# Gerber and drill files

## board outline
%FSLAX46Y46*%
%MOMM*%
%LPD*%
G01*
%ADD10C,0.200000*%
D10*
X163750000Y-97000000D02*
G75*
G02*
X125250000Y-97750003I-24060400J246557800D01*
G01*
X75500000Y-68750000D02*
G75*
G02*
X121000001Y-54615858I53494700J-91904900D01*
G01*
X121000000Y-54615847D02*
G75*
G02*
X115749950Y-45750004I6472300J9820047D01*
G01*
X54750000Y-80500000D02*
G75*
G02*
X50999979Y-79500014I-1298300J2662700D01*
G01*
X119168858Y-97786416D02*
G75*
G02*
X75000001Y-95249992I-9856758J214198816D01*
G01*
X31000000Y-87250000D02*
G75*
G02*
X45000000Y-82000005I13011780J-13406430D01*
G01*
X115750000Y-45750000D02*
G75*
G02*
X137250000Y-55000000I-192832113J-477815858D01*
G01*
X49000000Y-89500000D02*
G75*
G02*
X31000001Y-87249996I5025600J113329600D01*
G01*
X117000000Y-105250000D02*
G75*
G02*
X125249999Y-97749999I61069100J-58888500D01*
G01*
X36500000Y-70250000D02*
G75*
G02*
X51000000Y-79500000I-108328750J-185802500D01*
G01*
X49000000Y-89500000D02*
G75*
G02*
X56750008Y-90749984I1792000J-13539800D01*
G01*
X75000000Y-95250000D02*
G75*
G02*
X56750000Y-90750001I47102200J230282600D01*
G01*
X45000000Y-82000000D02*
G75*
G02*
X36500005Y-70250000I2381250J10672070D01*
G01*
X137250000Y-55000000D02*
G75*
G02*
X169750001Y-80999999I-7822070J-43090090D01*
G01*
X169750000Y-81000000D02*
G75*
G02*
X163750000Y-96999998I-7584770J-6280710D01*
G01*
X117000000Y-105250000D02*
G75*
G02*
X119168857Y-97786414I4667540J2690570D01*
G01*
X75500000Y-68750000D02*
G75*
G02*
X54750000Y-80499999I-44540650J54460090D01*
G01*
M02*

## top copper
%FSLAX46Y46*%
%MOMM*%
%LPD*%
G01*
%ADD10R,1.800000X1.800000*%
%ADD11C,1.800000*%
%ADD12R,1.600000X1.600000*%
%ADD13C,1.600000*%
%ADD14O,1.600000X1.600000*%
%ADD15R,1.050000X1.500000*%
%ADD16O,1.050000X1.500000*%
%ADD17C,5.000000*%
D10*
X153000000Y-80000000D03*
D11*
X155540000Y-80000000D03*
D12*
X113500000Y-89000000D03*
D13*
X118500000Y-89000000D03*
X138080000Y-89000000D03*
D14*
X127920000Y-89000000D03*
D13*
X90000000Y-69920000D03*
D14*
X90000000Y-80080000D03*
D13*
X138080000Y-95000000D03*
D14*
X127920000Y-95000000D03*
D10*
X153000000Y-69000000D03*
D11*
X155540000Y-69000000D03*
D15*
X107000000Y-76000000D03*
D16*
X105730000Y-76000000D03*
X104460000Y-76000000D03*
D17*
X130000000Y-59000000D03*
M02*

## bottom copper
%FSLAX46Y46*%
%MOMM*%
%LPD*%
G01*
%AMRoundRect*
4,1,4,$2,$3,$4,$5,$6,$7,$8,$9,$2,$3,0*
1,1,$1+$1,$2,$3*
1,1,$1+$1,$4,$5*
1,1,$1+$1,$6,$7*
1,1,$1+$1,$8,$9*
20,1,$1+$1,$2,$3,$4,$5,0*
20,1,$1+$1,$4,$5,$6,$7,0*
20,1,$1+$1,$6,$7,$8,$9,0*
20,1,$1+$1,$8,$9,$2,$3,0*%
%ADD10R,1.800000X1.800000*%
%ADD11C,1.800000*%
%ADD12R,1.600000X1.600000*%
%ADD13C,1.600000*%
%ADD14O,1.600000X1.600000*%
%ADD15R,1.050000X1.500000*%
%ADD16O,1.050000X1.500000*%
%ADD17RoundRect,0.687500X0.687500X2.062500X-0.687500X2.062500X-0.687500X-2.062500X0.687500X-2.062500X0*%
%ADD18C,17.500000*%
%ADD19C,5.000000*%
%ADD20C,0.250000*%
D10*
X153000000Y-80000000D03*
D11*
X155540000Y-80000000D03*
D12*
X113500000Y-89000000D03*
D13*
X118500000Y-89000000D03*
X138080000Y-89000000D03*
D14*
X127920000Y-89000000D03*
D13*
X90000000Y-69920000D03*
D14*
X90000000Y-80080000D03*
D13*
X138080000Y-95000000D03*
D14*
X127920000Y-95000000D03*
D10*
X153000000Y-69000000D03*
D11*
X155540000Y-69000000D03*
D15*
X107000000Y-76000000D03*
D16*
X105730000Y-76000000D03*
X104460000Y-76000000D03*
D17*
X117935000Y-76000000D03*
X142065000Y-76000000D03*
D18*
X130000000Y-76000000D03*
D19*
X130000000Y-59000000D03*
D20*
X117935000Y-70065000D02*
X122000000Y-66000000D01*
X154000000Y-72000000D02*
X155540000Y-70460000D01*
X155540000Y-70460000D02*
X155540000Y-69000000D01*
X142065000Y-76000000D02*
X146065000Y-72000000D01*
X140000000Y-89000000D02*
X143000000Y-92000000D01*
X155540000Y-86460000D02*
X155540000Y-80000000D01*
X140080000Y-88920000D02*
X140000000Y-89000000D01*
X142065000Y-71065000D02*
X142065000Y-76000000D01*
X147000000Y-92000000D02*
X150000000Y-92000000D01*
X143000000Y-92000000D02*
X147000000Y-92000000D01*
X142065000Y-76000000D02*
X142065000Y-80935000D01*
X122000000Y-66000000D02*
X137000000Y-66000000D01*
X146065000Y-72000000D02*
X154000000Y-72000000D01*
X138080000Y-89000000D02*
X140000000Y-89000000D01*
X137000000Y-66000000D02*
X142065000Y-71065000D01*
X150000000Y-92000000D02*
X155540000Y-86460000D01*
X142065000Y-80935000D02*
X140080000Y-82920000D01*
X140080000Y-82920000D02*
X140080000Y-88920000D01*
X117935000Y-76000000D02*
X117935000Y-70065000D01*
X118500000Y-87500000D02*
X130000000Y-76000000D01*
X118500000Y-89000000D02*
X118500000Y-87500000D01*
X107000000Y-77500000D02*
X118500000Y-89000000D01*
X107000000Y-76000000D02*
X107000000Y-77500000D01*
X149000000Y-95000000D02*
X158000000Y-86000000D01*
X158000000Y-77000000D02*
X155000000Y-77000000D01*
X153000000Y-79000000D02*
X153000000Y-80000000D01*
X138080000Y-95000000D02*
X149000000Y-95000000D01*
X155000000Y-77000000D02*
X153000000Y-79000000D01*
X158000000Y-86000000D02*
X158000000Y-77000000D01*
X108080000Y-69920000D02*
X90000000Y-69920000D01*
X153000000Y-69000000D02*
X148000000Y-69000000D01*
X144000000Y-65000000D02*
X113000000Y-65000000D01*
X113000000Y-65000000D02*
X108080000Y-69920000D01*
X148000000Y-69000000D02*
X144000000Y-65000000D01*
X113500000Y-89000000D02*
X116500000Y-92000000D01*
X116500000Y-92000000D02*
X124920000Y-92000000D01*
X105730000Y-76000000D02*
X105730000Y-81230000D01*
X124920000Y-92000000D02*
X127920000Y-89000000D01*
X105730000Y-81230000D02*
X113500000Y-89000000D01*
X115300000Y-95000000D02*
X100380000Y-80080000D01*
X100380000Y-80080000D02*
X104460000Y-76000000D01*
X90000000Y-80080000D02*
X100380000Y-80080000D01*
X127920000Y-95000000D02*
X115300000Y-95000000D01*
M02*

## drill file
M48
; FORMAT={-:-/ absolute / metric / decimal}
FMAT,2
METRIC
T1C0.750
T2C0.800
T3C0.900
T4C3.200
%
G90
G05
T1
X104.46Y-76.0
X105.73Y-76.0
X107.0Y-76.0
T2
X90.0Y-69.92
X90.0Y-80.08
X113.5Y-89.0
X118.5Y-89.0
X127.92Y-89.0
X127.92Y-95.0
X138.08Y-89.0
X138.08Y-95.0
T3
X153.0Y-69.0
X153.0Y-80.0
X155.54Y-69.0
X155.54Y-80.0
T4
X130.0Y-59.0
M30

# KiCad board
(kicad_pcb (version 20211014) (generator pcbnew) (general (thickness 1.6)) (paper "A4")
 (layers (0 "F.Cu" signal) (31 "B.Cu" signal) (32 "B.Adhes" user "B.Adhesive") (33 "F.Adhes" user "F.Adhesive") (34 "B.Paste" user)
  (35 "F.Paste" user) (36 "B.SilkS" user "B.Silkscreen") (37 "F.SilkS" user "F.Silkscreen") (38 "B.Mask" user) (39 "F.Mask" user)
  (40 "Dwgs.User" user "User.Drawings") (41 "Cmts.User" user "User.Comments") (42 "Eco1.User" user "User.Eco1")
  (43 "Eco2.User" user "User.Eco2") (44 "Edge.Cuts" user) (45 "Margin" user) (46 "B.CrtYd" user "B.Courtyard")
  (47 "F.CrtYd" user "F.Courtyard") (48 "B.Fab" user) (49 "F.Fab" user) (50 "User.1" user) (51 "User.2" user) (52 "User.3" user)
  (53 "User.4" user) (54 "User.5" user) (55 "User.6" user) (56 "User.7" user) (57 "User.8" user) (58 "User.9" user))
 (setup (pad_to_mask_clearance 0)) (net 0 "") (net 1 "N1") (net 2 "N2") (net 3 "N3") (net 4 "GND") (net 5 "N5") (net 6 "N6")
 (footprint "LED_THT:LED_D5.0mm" (layer "F.Cu") (at 153 80)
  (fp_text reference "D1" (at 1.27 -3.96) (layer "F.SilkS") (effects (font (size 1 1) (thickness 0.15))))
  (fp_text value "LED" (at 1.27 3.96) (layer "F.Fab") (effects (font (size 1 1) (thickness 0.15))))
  (pad "1" thru_hole rect (at 0 0) (size 1.8 1.8) (drill 0.9) (layers *.Cu *.Mask) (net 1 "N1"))
  (pad "2" thru_hole circle (at 2.54 0) (size 1.8 1.8) (drill 0.9) (layers *.Cu *.Mask) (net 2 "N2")))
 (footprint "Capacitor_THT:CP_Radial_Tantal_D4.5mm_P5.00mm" (layer "F.Cu") (at 113.5 89)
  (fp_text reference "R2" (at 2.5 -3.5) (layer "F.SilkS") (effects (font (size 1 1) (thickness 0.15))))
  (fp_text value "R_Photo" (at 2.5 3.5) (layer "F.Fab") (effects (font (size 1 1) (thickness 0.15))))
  (pad "1" thru_hole rect (at 0 0) (size 1.6 1.6) (drill 0.8) (layers *.Cu *.Mask) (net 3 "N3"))
  (pad "2" thru_hole circle (at 5 0) (size 1.6 1.6) (drill 0.8) (layers *.Cu *.Mask) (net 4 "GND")))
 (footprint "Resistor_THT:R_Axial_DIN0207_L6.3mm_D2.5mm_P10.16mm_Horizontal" (layer "F.Cu") (at 138.08 89 180)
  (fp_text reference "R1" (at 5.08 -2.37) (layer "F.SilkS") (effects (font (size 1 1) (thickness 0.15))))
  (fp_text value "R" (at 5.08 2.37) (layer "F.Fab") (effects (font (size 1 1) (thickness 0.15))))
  (pad "1" thru_hole circle (at 0 0 180) (size 1.6 1.6) (drill 0.8) (layers *.Cu *.Mask) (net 2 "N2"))
  (pad "2" thru_hole oval (at 10.16 0 180) (size 1.6 1.6) (drill 0.8) (layers *.Cu *.Mask) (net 3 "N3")))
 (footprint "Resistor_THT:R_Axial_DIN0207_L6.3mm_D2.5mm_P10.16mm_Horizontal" (layer "F.Cu") (at 90 69.92 -90)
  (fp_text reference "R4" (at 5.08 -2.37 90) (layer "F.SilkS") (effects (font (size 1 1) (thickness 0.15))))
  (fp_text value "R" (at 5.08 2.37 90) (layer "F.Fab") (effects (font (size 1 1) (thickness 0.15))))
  (pad "1" thru_hole circle (at 0 0 270) (size 1.6 1.6) (drill 0.8) (layers *.Cu *.Mask) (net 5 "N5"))
  (pad "2" thru_hole oval (at 10.16 0 270) (size 1.6 1.6) (drill 0.8) (layers *.Cu *.Mask) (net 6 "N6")))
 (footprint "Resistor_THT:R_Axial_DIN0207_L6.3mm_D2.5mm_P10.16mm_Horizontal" (layer "F.Cu") (at 138.08 95 180)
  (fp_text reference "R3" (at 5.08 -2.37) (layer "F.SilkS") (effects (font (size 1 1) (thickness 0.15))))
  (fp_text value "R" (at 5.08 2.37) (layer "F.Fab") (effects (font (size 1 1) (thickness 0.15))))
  (pad "1" thru_hole circle (at 0 0 180) (size 1.6 1.6) (drill 0.8) (layers *.Cu *.Mask) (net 1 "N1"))
  (pad "2" thru_hole oval (at 10.16 0 180) (size 1.6 1.6) (drill 0.8) (layers *.Cu *.Mask) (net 6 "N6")))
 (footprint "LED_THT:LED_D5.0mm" (layer "F.Cu") (at 153 69)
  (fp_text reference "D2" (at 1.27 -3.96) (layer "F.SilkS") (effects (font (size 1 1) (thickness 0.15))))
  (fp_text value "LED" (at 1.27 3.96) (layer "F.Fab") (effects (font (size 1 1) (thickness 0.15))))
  (pad "1" thru_hole rect (at 0 0) (size 1.8 1.8) (drill 0.9) (layers *.Cu *.Mask) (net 5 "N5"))
  (pad "2" thru_hole circle (at 2.54 0) (size 1.8 1.8) (drill 0.9) (layers *.Cu *.Mask) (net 2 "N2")))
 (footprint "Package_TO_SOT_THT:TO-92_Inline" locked (layer "F.Cu") (at 107 76 180)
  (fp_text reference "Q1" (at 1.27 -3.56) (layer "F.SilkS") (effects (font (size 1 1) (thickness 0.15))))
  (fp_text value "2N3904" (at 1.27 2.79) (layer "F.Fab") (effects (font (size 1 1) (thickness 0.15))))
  (pad "1" thru_hole rect locked (at 0 0 180) (size 1.05 1.5) (drill 0.75) (layers *.Cu *.Mask) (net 4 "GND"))
  (pad "2" thru_hole oval locked (at 1.27 0 180) (size 1.05 1.5) (drill 0.75) (layers *.Cu *.Mask) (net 3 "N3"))
  (pad "3" thru_hole oval locked (at 2.54 0 180) (size 1.05 1.5) (drill 0.75) (layers *.Cu *.Mask) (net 6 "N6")))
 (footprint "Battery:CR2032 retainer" (layer "B.Cu") (at 130 76 180)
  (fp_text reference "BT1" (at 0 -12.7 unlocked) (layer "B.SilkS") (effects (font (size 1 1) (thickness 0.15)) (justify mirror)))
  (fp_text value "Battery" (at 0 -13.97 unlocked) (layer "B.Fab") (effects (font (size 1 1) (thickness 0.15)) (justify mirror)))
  (pad "1" smd roundrect (at 12.065 0 180) (size 2.75 5.5) (layers "B.Cu" "B.Paste" "B.Mask") (roundrect_rratio 0.25) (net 2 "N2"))
  (pad "1" smd roundrect (at -12.065 0 180) (size 2.75 5.5) (layers "B.Cu" "B.Paste" "B.Mask") (roundrect_rratio 0.25) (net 2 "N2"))
  (pad "2" smd circle (at 0 0 180) (size 17.5 17.5) (layers "B.Cu" "B.Paste" "B.Mask") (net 4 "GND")))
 (gr_arc (start 163.75 97) (mid 144.514595 98.124194) (end 125.25 97.75) (layer "Edge.Cuts") (width 0.2))
 (gr_arc (start 75.5 68.75) (mid 97.448224 59.101885) (end 121 54.615847) (layer "Edge.Cuts") (width 0.2))
 (gr_arc (start 121 54.615847) (mid 117.352438 50.788445) (end 115.75 45.75) (layer "Edge.Cuts") (width 0.2))
 (gr_arc (start 54.75 80.5) (mid 52.675705 80.696188) (end 51 79.5) (layer "Edge.Cuts") (width 0.2))
 (gr_arc (start 119.168858 97.786416) (mid 97.018838 97.660405) (end 75 95.25) (layer "Edge.Cuts") (width 0.2))
 (gr_arc (start 31 87.25) (mid 37.451893 83.163381) (end 45 82) (layer "Edge.Cuts") (width 0.2))
 (gr_arc (start 115.75 45.75) (mid 126.552529 50.252906) (end 137.25 55) (layer "Edge.Cuts") (width 0.2))
 (gr_arc (start 49 89.5) (mid 39.954954 88.735369) (end 31 87.25) (layer "Edge.Cuts") (width 0.2))
 (gr_arc (start 117 105.25) (mid 121.001657 101.364323) (end 125.25 97.75) (layer "Edge.Cuts") (width 0.2))
 (gr_arc (start 36.5 70.25) (mid 43.8425 74.73) (end 51 79.5) (layer "Edge.Cuts") (width 0.2))
 (gr_arc (start 49 89.5) (mid 52.966743 89.556192) (end 56.75 90.75) (layer "Edge.Cuts") (width 0.2))
 (gr_arc (start 75 95.25) (mid 65.83 93.182501) (end 56.75 90.75) (layer "Edge.Cuts") (width 0.2))
 (gr_arc (start 45 82) (mid 38.521842 77.736859) (end 36.5 70.25) (layer "Edge.Cuts") (width 0.2))
 (gr_arc (start 137.25 55) (mid 156.78601 63.892488) (end 169.75 81) (layer "Edge.Cuts") (width 0.2))
 (gr_arc (start 169.75 81) (mid 171.385868 90.73845) (end 163.75 97) (layer "Edge.Cuts") (width 0.2))
 (gr_arc (start 117 105.25) (mid 116.494053 101.056057) (end 119.168858 97.786416) (layer "Edge.Cuts") (width 0.2))
 (gr_arc (start 75.5 68.75) (mid 65.626442 75.510525) (end 54.75 80.5) (layer "Edge.Cuts") (width 0.2))
 (via (at 130 59) (size 5) (drill 3.2) (layers "F.Cu" "B.Cu") (free) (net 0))
 (segment (start 117.935 70.065) (end 122 66) (width 0.25) (layer "B.Cu") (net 2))
 (segment (start 154 72) (end 155.54 70.46) (width 0.25) (layer "B.Cu") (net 2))
 (segment (start 155.54 70.46) (end 155.54 69) (width 0.25) (layer "B.Cu") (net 2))
 (segment (start 142.065 76) (end 146.065 72) (width 0.25) (layer "B.Cu") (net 2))
 (segment (start 140 89) (end 143 92) (width 0.25) (layer "B.Cu") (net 2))
 (segment (start 155.54 86.46) (end 155.54 80) (width 0.25) (layer "B.Cu") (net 2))
 (segment (start 140.08 88.92) (end 140 89) (width 0.25) (layer "B.Cu") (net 2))
 (segment (start 142.065 71.065) (end 142.065 76) (width 0.25) (layer "B.Cu") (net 2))
 (segment (start 147 92) (end 150 92) (width 0.25) (layer "B.Cu") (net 2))
 (segment (start 143 92) (end 147 92) (width 0.25) (layer "B.Cu") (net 2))
 (segment (start 142.065 76) (end 142.065 80.935) (width 0.25) (layer "B.Cu") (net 2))
 (segment (start 122 66) (end 137 66) (width 0.25) (layer "B.Cu") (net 2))
 (segment (start 146.065 72) (end 154 72) (width 0.25) (layer "B.Cu") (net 2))
 (segment (start 138.08 89) (end 140 89) (width 0.25) (layer "B.Cu") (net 2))
 (segment (start 137 66) (end 142.065 71.065) (width 0.25) (layer "B.Cu") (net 2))
 (segment (start 150 92) (end 155.54 86.46) (width 0.25) (layer "B.Cu") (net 2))
 (segment (start 142.065 80.935) (end 140.08 82.92) (width 0.25) (layer "B.Cu") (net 2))
 (segment (start 140.08 82.92) (end 140.08 88.92) (width 0.25) (layer "B.Cu") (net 2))
 (segment (start 117.935 76) (end 117.935 70.065) (width 0.25) (layer "B.Cu") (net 2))
 (segment (start 118.5 87.5) (end 130 76) (width 0.25) (layer "B.Cu") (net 4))
 (segment (start 118.5 89) (end 118.5 87.5) (width 0.25) (layer "B.Cu") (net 4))
 (segment (start 107 77.5) (end 118.5 89) (width 0.25) (layer "B.Cu") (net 4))
 (segment (start 107 76) (end 107 77.5) (width 0.25) (layer "B.Cu") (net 4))
 (segment (start 149 95) (end 158 86) (width 0.25) (layer "B.Cu") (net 1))
 (segment (start 158 77) (end 155 77) (width 0.25) (layer "B.Cu") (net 1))
 (segment (start 153 79) (end 153 80) (width 0.25) (layer "B.Cu") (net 1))
 (segment (start 138.08 95) (end 149 95) (width 0.25) (layer "B.Cu") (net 1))
 (segment (start 155 77) (end 153 79) (width 0.25) (layer "B.Cu") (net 1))
 (segment (start 158 86) (end 158 77) (width 0.25) (layer "B.Cu") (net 1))
 (segment (start 108.08 69.92) (end 90 69.92) (width 0.25) (layer "B.Cu") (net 5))
 (segment (start 153 69) (end 148 69) (width 0.25) (layer "B.Cu") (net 5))
 (segment (start 144 65) (end 113 65) (width 0.25) (layer "B.Cu") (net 5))
 (segment (start 113 65) (end 108.08 69.92) (width 0.25) (layer "B.Cu") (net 5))
 (segment (start 148 69) (end 144 65) (width 0.25) (layer "B.Cu") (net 5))
 (segment (start 113.5 89) (end 116.5 92) (width 0.25) (layer "B.Cu") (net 3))
 (segment (start 116.5 92) (end 124.92 92) (width 0.25) (layer "B.Cu") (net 3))
 (segment (start 105.73 76) (end 105.73 81.23) (width 0.25) (layer "B.Cu") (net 3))
 (segment (start 124.92 92) (end 127.92 89) (width 0.25) (layer "B.Cu") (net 3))
 (segment (start 105.73 81.23) (end 113.5 89) (width 0.25) (layer "B.Cu") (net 3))
 (segment (start 115.3 95) (end 100.38 80.08) (width 0.25) (layer "B.Cu") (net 6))
 (segment (start 100.38 80.08) (end 104.46 76) (width 0.25) (layer "B.Cu") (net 6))
 (segment (start 90 80.08) (end 100.38 80.08) (width 0.25) (layer "B.Cu") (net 6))
 (segment (start 127.92 95) (end 115.3 95) (width 0.25) (layer "B.Cu") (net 6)))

